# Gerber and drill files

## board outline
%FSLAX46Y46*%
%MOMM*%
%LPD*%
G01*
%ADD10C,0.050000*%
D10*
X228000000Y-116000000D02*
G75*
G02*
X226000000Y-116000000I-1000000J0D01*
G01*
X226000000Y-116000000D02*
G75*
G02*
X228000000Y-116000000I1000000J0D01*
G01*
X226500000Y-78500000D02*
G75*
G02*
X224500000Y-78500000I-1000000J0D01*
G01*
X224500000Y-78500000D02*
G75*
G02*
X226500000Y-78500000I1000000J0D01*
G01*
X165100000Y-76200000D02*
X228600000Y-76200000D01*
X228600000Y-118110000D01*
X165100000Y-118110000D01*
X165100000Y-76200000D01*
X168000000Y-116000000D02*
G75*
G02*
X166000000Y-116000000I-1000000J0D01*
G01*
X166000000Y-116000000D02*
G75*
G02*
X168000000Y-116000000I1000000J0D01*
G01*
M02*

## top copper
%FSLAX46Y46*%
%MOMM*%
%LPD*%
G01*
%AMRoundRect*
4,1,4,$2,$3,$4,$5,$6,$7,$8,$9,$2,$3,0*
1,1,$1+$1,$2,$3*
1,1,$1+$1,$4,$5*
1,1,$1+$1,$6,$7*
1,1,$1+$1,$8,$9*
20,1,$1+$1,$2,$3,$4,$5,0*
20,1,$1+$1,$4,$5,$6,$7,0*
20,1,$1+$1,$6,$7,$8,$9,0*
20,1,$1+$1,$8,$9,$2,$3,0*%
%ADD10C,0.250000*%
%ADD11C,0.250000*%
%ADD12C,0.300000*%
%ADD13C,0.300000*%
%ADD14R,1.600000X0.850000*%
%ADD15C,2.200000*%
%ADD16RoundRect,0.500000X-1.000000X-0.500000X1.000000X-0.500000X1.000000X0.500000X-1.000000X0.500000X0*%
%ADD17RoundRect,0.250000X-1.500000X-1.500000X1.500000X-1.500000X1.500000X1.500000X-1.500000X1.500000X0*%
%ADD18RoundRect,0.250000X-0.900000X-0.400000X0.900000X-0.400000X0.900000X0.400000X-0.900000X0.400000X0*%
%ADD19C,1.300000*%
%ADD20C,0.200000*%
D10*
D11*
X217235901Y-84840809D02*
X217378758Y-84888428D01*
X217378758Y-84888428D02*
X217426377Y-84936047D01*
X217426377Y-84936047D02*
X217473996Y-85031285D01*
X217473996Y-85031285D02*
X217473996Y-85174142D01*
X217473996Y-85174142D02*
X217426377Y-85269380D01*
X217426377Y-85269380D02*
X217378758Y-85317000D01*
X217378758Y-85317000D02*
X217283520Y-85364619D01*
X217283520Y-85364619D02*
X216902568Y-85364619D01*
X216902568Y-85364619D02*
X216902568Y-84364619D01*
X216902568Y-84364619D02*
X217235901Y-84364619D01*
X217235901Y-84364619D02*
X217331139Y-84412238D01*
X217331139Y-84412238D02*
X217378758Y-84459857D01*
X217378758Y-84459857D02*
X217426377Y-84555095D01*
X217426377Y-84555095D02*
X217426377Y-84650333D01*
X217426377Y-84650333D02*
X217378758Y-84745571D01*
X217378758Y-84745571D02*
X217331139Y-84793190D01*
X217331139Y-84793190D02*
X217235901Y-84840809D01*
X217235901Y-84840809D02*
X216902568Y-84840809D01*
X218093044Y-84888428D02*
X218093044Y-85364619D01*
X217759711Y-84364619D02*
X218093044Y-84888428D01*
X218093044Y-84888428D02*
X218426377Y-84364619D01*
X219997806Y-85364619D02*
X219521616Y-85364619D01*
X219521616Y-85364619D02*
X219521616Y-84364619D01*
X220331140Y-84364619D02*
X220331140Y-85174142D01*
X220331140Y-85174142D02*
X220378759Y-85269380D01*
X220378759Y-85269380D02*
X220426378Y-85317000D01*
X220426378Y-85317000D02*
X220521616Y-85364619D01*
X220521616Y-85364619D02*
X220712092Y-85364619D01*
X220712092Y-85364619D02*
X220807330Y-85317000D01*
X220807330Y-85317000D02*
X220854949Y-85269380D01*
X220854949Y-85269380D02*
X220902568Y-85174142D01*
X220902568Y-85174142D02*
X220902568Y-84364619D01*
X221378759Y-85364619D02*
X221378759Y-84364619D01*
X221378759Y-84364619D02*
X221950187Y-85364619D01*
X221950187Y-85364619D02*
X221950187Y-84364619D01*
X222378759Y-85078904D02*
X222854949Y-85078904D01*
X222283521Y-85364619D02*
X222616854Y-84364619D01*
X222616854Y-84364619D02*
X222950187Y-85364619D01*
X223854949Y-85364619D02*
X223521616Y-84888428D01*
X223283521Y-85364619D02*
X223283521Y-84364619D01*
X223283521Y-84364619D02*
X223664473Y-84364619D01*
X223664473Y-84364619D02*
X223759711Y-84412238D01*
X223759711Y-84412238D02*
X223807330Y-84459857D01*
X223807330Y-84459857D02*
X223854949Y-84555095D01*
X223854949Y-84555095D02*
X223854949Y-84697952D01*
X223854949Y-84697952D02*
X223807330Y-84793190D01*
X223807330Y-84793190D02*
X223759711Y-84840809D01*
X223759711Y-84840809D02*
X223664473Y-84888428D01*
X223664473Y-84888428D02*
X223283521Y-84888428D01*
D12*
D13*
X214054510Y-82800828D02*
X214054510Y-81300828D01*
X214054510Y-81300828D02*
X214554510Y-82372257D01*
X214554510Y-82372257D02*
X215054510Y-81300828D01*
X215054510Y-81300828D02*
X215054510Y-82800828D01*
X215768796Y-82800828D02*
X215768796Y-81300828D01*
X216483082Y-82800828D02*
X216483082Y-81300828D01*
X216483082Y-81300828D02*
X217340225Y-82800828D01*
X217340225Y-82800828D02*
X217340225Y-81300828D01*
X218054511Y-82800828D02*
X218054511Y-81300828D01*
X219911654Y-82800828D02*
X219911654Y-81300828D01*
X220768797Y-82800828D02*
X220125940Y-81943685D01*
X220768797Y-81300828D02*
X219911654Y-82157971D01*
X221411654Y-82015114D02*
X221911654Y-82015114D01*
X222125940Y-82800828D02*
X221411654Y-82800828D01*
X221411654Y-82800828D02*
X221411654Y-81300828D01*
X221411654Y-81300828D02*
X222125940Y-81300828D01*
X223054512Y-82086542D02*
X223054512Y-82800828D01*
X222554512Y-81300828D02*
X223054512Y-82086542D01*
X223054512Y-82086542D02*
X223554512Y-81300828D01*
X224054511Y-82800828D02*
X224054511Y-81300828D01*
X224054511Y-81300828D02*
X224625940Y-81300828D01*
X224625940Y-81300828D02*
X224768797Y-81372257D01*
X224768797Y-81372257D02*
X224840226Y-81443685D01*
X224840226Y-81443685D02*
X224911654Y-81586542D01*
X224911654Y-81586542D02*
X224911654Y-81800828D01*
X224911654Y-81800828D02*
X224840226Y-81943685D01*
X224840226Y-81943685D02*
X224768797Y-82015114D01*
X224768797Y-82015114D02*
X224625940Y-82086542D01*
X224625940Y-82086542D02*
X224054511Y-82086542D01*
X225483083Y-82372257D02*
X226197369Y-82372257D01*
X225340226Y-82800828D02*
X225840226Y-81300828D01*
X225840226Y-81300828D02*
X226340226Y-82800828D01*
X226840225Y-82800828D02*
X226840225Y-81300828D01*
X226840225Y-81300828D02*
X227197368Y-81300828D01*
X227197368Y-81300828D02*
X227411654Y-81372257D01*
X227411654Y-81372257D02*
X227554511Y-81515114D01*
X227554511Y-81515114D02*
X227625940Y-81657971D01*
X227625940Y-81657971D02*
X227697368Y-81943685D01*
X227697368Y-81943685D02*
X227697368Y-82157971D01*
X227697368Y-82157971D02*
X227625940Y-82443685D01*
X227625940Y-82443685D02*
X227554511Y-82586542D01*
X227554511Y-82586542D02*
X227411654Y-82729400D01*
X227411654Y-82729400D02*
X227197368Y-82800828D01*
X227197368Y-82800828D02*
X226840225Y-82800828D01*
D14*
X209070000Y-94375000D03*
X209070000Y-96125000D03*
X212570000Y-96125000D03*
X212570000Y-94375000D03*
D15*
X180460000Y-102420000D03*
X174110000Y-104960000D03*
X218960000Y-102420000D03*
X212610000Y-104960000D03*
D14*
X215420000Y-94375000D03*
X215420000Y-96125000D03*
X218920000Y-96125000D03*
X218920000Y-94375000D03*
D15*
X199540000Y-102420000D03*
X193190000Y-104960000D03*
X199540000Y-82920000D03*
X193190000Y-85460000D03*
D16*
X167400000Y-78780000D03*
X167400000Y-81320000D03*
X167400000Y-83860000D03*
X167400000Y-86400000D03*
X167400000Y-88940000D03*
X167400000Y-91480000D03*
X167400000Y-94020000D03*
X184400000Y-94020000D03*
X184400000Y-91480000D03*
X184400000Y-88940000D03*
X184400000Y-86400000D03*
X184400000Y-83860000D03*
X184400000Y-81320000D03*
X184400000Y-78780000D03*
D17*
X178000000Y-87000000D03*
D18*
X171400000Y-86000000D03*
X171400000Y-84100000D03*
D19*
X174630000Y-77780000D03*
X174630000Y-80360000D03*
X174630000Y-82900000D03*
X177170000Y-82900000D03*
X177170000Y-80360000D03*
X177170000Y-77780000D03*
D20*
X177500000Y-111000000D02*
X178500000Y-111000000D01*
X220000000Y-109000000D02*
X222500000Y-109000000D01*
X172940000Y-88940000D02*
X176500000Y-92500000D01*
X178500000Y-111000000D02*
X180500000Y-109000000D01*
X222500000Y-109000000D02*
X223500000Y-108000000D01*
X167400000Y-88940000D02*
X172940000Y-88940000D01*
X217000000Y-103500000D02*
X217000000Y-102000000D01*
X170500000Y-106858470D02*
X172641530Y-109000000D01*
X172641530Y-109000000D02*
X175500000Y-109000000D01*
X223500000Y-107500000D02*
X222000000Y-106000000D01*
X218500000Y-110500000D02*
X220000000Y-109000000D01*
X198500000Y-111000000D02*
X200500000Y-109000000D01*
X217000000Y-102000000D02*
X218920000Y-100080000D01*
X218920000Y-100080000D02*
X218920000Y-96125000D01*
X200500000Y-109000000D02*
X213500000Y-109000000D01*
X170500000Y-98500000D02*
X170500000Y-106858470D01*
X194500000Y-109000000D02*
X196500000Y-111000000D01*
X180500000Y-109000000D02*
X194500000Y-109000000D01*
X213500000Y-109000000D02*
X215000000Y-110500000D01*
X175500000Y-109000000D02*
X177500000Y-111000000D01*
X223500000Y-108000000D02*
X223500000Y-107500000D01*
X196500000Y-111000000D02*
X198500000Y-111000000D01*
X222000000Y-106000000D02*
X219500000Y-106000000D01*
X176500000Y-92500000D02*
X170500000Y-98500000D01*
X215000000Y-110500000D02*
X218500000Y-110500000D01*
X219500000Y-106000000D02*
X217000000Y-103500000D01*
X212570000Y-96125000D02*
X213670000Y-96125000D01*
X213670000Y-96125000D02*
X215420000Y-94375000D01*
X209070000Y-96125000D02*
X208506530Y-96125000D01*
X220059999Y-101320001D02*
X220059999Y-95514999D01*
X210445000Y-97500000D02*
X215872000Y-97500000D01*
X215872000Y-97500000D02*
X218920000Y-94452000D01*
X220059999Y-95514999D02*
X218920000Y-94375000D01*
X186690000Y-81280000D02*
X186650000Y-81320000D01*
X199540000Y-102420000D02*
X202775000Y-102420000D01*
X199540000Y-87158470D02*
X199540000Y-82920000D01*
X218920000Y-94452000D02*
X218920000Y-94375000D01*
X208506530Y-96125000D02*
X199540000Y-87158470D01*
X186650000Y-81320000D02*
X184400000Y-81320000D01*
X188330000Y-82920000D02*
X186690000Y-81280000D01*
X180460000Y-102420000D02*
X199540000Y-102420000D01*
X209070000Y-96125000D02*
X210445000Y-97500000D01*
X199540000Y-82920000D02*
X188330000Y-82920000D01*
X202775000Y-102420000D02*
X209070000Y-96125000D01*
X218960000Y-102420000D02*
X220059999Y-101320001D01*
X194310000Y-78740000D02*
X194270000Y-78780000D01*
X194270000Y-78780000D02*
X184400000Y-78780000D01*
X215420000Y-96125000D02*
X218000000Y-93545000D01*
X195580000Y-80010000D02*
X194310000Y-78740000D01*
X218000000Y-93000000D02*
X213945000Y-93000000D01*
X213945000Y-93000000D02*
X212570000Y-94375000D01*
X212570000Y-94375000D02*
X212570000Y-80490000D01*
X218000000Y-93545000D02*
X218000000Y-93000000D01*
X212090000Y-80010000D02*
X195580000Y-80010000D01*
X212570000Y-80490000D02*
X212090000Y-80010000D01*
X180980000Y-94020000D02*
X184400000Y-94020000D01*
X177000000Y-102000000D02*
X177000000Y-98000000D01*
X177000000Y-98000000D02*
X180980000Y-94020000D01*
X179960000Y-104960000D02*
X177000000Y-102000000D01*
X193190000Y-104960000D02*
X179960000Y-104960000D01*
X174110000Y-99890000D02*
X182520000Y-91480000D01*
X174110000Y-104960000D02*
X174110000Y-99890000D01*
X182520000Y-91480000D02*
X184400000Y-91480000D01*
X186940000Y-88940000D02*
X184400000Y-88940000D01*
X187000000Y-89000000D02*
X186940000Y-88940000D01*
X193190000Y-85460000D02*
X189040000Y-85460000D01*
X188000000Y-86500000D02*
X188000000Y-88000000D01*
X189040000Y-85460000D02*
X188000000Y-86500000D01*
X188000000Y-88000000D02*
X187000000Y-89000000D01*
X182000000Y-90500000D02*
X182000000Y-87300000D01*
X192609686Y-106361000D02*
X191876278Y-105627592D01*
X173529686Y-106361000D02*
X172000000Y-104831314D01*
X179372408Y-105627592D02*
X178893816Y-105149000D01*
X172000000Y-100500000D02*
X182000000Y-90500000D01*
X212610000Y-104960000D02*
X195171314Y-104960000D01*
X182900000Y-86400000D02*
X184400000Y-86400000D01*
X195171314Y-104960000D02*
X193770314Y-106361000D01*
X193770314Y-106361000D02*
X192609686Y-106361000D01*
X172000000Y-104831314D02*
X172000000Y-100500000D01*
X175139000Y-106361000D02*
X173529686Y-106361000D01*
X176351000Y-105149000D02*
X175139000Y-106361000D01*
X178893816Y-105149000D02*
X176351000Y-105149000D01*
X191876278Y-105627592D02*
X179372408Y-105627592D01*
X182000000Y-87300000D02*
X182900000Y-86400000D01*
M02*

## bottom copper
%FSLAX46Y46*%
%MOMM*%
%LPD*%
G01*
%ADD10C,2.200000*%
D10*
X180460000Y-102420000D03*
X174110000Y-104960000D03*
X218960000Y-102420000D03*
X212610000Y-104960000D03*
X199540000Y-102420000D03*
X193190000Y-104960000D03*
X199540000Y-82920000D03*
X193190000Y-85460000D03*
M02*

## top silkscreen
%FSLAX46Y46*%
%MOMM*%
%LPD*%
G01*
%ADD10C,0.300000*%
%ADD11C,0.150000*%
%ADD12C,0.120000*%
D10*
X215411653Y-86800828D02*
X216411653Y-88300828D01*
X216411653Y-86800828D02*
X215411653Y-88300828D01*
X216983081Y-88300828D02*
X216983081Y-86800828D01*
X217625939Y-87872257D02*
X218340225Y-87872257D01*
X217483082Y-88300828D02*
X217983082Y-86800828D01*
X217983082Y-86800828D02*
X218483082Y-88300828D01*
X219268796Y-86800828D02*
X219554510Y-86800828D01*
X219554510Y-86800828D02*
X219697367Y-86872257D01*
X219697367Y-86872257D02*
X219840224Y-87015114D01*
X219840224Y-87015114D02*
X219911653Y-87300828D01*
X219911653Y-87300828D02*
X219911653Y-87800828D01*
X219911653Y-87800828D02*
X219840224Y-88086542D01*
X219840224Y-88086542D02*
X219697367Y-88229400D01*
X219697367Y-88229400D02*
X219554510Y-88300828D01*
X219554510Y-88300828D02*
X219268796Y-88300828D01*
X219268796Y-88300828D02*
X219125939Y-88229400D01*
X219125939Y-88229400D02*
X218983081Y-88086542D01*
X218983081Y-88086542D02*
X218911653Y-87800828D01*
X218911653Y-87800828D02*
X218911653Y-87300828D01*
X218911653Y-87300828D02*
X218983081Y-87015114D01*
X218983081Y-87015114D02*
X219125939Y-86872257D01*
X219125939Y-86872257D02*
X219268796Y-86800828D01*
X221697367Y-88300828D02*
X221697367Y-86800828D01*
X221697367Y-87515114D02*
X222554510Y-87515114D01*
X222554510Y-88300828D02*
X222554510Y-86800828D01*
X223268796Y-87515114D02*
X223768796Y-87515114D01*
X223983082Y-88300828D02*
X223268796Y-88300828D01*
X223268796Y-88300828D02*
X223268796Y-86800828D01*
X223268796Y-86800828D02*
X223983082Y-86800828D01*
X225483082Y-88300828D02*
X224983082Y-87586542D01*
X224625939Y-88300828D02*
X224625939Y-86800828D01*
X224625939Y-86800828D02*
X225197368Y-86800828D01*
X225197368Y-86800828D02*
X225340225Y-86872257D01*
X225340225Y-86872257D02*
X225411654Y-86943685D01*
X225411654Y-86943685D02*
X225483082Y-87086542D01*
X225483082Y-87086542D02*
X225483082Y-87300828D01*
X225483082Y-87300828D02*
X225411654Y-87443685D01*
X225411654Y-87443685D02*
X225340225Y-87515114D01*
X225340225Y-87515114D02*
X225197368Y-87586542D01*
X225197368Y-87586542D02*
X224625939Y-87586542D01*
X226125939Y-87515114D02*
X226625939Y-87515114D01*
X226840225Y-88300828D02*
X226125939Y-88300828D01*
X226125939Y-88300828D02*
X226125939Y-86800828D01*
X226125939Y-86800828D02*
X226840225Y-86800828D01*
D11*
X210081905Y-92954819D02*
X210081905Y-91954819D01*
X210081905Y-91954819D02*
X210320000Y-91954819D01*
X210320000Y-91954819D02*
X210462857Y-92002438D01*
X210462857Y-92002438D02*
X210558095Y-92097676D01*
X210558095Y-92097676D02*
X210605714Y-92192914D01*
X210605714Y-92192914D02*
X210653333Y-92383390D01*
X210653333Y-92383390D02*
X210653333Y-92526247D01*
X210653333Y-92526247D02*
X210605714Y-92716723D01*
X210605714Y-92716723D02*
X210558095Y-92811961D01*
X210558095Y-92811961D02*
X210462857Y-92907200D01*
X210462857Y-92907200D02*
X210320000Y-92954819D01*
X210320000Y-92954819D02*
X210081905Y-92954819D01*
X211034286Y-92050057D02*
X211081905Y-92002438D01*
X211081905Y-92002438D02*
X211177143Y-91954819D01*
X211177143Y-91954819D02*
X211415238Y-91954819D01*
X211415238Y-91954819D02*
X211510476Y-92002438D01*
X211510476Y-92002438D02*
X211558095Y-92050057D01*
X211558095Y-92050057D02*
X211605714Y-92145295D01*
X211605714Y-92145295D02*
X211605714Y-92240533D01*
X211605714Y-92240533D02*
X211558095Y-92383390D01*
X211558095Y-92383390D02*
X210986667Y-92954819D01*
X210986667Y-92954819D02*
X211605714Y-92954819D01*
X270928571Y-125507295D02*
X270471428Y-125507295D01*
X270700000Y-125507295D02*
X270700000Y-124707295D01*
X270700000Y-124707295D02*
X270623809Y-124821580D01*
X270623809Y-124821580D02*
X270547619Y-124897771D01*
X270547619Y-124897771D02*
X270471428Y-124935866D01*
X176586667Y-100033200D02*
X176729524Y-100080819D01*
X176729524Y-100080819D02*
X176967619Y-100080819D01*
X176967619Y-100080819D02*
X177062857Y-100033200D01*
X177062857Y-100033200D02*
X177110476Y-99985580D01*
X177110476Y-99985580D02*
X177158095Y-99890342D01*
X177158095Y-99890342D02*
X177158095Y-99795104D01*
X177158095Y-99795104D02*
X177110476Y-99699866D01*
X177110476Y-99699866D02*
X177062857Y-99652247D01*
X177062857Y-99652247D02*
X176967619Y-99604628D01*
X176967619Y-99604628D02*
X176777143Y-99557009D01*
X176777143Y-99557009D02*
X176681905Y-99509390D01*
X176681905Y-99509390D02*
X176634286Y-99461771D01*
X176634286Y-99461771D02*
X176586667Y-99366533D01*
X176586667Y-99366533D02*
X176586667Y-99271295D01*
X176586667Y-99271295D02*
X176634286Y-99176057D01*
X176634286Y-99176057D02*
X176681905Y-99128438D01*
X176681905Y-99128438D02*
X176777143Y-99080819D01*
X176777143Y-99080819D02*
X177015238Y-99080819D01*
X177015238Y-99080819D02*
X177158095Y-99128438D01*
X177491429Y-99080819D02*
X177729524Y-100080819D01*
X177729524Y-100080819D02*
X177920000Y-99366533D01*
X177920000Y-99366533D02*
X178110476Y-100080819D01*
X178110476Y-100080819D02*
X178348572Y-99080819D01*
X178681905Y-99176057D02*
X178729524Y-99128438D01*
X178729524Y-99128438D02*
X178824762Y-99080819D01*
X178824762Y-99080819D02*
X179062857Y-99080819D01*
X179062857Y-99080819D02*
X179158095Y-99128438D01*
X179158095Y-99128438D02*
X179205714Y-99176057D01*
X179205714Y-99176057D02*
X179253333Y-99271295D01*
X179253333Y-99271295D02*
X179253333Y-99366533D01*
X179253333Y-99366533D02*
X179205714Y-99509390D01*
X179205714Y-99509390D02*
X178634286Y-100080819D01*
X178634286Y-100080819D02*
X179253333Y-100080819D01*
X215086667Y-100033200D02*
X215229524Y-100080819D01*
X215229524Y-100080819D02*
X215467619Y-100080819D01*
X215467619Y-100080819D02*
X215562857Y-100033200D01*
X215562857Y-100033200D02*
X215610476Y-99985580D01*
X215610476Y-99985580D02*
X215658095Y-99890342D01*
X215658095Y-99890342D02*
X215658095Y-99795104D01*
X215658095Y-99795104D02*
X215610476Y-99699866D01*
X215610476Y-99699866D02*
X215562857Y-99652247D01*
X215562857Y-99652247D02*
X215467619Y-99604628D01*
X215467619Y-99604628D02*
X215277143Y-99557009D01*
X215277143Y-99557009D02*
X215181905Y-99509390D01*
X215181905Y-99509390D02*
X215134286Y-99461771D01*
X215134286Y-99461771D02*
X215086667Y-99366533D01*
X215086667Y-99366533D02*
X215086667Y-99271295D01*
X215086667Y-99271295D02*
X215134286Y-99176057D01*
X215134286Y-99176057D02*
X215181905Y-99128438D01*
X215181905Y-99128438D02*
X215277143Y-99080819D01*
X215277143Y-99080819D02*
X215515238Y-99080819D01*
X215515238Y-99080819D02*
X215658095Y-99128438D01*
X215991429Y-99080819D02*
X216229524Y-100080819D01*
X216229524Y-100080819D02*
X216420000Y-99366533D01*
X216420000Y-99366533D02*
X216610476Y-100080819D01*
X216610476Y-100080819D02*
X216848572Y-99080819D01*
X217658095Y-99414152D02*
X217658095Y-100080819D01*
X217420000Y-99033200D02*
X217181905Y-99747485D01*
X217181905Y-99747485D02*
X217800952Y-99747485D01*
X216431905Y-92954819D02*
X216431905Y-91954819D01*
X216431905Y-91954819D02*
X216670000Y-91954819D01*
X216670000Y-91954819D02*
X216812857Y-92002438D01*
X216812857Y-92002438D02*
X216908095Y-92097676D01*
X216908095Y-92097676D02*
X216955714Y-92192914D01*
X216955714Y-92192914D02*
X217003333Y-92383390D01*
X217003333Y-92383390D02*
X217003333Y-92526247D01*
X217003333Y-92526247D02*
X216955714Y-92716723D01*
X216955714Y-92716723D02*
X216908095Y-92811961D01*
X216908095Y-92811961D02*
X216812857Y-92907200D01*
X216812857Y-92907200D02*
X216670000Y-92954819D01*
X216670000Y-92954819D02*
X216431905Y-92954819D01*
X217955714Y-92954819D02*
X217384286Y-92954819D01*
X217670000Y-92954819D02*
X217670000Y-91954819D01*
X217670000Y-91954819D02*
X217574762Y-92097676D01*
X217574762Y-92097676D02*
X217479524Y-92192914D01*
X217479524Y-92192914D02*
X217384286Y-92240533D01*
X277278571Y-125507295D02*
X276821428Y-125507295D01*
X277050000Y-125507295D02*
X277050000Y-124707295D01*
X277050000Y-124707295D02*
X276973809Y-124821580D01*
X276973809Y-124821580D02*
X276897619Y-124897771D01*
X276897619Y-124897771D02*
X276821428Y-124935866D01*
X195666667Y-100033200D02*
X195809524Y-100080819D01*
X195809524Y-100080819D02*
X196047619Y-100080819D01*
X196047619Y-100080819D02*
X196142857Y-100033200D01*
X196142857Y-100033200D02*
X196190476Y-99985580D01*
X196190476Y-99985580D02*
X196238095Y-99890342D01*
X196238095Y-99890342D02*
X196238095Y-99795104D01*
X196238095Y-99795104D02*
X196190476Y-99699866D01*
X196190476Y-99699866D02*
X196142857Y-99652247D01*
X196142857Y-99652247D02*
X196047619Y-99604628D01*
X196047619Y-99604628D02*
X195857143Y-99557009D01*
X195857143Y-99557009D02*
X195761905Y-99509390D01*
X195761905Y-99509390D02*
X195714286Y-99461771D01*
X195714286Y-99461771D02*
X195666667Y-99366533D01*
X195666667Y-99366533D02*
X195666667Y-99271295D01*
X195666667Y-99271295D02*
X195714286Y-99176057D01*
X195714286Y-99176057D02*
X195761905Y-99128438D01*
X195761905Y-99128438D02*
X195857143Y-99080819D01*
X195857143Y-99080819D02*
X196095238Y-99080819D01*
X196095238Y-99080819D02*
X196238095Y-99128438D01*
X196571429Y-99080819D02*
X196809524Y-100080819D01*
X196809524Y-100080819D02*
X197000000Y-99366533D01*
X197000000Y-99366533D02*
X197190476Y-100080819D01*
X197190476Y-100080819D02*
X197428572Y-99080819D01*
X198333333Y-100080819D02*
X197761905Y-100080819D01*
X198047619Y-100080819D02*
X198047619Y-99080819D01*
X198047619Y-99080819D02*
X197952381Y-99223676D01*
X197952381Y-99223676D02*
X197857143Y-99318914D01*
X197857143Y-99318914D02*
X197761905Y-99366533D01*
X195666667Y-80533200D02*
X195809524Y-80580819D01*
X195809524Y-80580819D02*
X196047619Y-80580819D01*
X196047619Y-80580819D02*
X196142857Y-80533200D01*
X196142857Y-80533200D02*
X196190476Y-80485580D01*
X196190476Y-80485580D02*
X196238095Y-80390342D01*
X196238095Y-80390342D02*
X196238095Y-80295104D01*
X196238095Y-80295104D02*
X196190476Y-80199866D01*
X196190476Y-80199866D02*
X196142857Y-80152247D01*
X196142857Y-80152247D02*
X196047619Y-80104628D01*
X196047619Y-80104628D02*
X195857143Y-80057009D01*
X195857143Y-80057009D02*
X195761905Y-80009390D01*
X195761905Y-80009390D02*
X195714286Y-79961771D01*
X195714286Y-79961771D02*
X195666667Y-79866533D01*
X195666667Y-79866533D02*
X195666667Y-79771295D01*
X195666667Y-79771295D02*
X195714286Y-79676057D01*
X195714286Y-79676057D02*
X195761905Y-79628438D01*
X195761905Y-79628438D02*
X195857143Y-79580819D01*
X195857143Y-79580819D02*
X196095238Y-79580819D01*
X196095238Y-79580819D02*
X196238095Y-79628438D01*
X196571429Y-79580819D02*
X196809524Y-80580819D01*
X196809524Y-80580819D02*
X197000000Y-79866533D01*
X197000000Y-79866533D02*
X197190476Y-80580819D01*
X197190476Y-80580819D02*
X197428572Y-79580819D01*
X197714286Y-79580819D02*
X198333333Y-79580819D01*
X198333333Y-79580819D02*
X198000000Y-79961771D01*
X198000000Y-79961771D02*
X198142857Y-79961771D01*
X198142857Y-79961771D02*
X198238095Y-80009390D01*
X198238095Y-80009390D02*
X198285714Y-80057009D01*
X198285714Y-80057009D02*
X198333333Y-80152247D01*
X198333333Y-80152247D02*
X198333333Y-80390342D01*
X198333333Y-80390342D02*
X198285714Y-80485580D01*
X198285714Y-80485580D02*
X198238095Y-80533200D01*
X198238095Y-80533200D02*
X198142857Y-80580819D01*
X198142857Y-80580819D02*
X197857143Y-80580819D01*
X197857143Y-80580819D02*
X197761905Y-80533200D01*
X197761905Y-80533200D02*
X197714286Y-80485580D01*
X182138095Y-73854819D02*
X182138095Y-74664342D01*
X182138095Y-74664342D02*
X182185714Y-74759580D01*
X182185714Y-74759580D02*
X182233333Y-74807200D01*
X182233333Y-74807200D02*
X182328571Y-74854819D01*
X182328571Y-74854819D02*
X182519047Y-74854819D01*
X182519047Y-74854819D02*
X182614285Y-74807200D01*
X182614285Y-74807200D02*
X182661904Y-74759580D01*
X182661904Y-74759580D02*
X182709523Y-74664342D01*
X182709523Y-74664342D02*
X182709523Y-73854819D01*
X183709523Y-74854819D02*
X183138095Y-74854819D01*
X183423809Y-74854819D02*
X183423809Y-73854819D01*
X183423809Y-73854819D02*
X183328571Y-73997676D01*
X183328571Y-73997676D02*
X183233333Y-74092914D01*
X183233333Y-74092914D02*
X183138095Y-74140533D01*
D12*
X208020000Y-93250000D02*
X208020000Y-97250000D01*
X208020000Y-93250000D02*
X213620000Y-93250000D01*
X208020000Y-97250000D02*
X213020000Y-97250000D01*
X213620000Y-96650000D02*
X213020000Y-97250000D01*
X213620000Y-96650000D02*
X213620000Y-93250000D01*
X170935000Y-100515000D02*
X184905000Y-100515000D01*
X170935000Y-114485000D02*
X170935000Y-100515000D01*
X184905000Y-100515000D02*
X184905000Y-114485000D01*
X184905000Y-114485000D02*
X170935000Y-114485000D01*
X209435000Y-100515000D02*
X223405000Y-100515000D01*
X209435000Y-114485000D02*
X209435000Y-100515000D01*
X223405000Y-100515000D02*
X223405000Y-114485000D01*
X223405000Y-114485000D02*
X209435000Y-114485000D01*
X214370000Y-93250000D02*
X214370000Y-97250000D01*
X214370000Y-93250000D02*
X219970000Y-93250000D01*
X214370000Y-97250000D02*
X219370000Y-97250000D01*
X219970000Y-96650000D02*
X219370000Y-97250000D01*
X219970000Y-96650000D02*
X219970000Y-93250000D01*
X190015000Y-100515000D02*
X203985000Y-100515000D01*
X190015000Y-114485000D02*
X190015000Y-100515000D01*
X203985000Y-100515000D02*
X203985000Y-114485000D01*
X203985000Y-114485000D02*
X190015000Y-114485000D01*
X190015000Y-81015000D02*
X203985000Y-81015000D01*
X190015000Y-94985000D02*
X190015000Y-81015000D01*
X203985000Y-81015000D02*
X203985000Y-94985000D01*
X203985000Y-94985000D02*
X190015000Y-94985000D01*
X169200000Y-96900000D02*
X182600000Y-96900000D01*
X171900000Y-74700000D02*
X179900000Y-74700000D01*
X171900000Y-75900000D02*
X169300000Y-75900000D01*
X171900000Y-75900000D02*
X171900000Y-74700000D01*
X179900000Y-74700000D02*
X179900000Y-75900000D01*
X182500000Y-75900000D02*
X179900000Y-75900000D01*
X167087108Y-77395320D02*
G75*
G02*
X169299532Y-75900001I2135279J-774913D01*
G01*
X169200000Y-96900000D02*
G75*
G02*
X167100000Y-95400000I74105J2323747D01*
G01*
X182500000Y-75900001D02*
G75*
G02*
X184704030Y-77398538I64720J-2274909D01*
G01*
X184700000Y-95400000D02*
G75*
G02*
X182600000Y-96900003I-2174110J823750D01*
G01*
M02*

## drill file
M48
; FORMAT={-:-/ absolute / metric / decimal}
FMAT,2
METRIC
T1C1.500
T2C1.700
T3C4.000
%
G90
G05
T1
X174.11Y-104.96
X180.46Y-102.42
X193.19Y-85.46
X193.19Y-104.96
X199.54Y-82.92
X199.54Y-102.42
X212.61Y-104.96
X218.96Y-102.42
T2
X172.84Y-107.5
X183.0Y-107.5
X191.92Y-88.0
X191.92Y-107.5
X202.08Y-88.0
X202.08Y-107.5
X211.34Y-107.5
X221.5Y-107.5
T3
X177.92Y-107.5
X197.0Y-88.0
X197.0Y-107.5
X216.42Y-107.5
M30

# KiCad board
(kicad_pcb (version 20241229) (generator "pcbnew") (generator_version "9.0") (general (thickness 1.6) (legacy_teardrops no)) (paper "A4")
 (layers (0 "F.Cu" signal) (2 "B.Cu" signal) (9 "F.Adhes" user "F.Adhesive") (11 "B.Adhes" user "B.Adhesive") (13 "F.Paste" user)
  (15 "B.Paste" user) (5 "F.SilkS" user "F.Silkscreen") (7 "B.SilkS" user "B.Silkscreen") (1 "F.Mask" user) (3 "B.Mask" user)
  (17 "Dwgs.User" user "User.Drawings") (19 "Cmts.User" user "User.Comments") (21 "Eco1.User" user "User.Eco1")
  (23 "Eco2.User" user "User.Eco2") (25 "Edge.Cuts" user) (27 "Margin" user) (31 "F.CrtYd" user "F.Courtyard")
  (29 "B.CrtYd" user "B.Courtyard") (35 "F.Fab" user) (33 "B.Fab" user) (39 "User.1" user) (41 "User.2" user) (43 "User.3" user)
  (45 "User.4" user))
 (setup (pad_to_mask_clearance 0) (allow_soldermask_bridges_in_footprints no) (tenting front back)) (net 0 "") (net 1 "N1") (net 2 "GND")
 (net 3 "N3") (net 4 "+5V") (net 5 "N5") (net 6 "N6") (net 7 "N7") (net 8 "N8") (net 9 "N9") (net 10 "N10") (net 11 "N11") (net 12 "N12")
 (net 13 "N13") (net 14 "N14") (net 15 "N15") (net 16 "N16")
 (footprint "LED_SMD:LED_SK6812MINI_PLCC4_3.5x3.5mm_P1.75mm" (layer "F.Cu") (at 210.82 95.25)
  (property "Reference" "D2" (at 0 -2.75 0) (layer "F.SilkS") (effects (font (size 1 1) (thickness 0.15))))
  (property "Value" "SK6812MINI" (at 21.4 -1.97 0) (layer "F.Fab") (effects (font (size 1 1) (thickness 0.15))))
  (fp_line (start -2.8 -2) (end -2.8 2) (stroke (width 0.12) (type default)) (layer "F.SilkS"))
  (fp_line (start -2.8 -2) (end 2.8 -2) (stroke (width 0.12) (type solid)) (layer "F.SilkS"))
  (fp_line (start -2.8 2) (end 2.2 2) (stroke (width 0.12) (type solid)) (layer "F.SilkS"))
  (fp_line (start 2.8 1.4) (end 2.2 2) (stroke (width 0.12) (type default)) (layer "F.SilkS"))
  (fp_line (start 2.8 1.4) (end 2.8 -2) (stroke (width 0.12) (type solid)) (layer "F.SilkS"))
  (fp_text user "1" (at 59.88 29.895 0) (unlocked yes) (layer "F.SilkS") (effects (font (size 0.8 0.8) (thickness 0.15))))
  (pad "1" smd rect (at -1.75 -0.875) (size 1.6 0.85) (layers "F.Cu" "F.Mask" "F.Paste") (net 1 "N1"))
  (pad "2" smd rect (at -1.75 0.875) (size 1.6 0.85) (layers "F.Cu" "F.Mask" "F.Paste") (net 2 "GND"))
  (pad "3" smd rect (at 1.75 0.875) (size 1.6 0.85) (layers "F.Cu" "F.Mask" "F.Paste") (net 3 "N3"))
  (pad "4" smd rect (at 1.75 -0.875) (size 1.6 0.85) (layers "F.Cu" "F.Mask" "F.Paste") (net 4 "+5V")))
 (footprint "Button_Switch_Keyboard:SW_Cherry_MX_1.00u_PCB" (layer "F.Cu") (at 180.46 102.42)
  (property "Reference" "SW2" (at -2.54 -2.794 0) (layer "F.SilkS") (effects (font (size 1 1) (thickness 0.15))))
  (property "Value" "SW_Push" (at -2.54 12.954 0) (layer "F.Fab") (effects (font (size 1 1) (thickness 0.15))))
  (fp_line (start -9.525 -1.905) (end 4.445 -1.905) (stroke (width 0.12) (type solid)) (layer "F.SilkS"))
  (fp_line (start -9.525 12.065) (end -9.525 -1.905) (stroke (width 0.12) (type solid)) (layer "F.SilkS"))
  (fp_line (start 4.445 -1.905) (end 4.445 12.065) (stroke (width 0.12) (type solid)) (layer "F.SilkS"))
  (fp_line (start 4.445 12.065) (end -9.525 12.065) (stroke (width 0.12) (type solid)) (layer "F.SilkS"))
  (pad "" np_thru_hole circle (at -7.62 5.08) (size 1.7 1.7) (drill 1.7) (layers "*.Cu" "*.Mask"))
  (pad "" np_thru_hole circle (at -2.54 5.08) (size 4 4) (drill 4) (layers "*.Cu" "*.Mask"))
  (pad "" np_thru_hole circle (at 2.54 5.08) (size 1.7 1.7) (drill 1.7) (layers "*.Cu" "*.Mask"))
  (pad "1" thru_hole circle (at 0 0) (size 2.2 2.2) (drill 1.5) (layers "*.Cu" "*.Mask") (remove_unused_layers no) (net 2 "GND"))
  (pad "2" thru_hole circle (at -6.35 2.54) (size 2.2 2.2) (drill 1.5) (layers "*.Cu" "*.Mask") (remove_unused_layers no) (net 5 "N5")))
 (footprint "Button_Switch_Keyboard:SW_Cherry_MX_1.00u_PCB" (layer "F.Cu") (at 218.96 102.42)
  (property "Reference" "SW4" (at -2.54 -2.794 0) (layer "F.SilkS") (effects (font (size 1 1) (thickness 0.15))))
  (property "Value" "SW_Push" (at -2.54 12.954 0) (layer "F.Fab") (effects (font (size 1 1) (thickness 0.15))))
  (fp_line (start -9.525 -1.905) (end 4.445 -1.905) (stroke (width 0.12) (type solid)) (layer "F.SilkS"))
  (fp_line (start -9.525 12.065) (end -9.525 -1.905) (stroke (width 0.12) (type solid)) (layer "F.SilkS"))
  (fp_line (start 4.445 -1.905) (end 4.445 12.065) (stroke (width 0.12) (type solid)) (layer "F.SilkS"))
  (fp_line (start 4.445 12.065) (end -9.525 12.065) (stroke (width 0.12) (type solid)) (layer "F.SilkS"))
  (pad "" np_thru_hole circle (at -7.62 5.08) (size 1.7 1.7) (drill 1.7) (layers "*.Cu" "*.Mask"))
  (pad "" np_thru_hole circle (at -2.54 5.08) (size 4 4) (drill 4) (layers "*.Cu" "*.Mask"))
  (pad "" np_thru_hole circle (at 2.54 5.08) (size 1.7 1.7) (drill 1.7) (layers "*.Cu" "*.Mask"))
  (pad "1" thru_hole circle (at 0 0) (size 2.2 2.2) (drill 1.5) (layers "*.Cu" "*.Mask") (remove_unused_layers no) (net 2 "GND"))
  (pad "2" thru_hole circle (at -6.35 2.54) (size 2.2 2.2) (drill 1.5) (layers "*.Cu" "*.Mask") (remove_unused_layers no) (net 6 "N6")))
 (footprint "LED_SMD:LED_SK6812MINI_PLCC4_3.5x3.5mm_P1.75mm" (layer "F.Cu") (at 217.17 95.25)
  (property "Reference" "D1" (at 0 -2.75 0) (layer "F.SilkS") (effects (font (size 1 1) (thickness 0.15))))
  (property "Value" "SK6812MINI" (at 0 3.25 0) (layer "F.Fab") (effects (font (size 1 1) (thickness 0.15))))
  (fp_line (start -2.8 -2) (end -2.8 2) (stroke (width 0.12) (type default)) (layer "F.SilkS"))
  (fp_line (start -2.8 -2) (end 2.8 -2) (stroke (width 0.12) (type solid)) (layer "F.SilkS"))
  (fp_line (start -2.8 2) (end 2.2 2) (stroke (width 0.12) (type solid)) (layer "F.SilkS"))
  (fp_line (start 2.8 1.4) (end 2.2 2) (stroke (width 0.12) (type default)) (layer "F.SilkS"))
  (fp_line (start 2.8 1.4) (end 2.8 -2) (stroke (width 0.12) (type solid)) (layer "F.SilkS"))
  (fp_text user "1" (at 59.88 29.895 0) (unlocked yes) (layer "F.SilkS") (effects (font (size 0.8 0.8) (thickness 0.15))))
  (pad "1" smd rect (at -1.75 -0.875) (size 1.6 0.85) (layers "F.Cu" "F.Mask" "F.Paste") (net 3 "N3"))
  (pad "2" smd rect (at -1.75 0.875) (size 1.6 0.85) (layers "F.Cu" "F.Mask" "F.Paste") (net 4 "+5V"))
  (pad "3" smd rect (at 1.75 0.875) (size 1.6 0.85) (layers "F.Cu" "F.Mask" "F.Paste") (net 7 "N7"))
  (pad "4" smd rect (at 1.75 -0.875) (size 1.6 0.85) (layers "F.Cu" "F.Mask" "F.Paste") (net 2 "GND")))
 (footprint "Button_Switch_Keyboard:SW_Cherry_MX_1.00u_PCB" (layer "F.Cu") (at 199.54 102.42)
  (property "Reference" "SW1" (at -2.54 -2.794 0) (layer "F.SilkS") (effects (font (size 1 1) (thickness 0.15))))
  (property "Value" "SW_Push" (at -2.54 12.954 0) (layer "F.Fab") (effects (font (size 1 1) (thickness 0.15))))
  (fp_line (start -9.525 -1.905) (end 4.445 -1.905) (stroke (width 0.12) (type solid)) (layer "F.SilkS"))
  (fp_line (start -9.525 12.065) (end -9.525 -1.905) (stroke (width 0.12) (type solid)) (layer "F.SilkS"))
  (fp_line (start 4.445 -1.905) (end 4.445 12.065) (stroke (width 0.12) (type solid)) (layer "F.SilkS"))
  (fp_line (start 4.445 12.065) (end -9.525 12.065) (stroke (width 0.12) (type solid)) (layer "F.SilkS"))
  (pad "" np_thru_hole circle (at -7.62 5.08) (size 1.7 1.7) (drill 1.7) (layers "*.Cu" "*.Mask"))
  (pad "" np_thru_hole circle (at -2.54 5.08) (size 4 4) (drill 4) (layers "*.Cu" "*.Mask"))
  (pad "" np_thru_hole circle (at 2.54 5.08) (size 1.7 1.7) (drill 1.7) (layers "*.Cu" "*.Mask"))
  (pad "1" thru_hole circle (at 0 0) (size 2.2 2.2) (drill 1.5) (layers "*.Cu" "*.Mask") (remove_unused_layers no) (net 2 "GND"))
  (pad "2" thru_hole circle (at -6.35 2.54) (size 2.2 2.2) (drill 1.5) (layers "*.Cu" "*.Mask") (remove_unused_layers no) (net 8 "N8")))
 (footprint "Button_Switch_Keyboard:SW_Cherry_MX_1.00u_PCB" (layer "F.Cu") (at 199.54 82.92)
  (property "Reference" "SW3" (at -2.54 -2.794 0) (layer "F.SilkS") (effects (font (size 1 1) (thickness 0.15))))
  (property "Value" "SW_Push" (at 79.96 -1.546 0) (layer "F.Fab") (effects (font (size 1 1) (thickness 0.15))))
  (fp_line (start -9.525 -1.905) (end 4.445 -1.905) (stroke (width 0.12) (type solid)) (layer "F.SilkS"))
  (fp_line (start -9.525 12.065) (end -9.525 -1.905) (stroke (width 0.12) (type solid)) (layer "F.SilkS"))
  (fp_line (start 4.445 -1.905) (end 4.445 12.065) (stroke (width 0.12) (type solid)) (layer "F.SilkS"))
  (fp_line (start 4.445 12.065) (end -9.525 12.065) (stroke (width 0.12) (type solid)) (layer "F.SilkS"))
  (pad "" np_thru_hole circle (at -7.62 5.08) (size 1.7 1.7) (drill 1.7) (layers "*.Cu" "*.Mask"))
  (pad "" np_thru_hole circle (at -2.54 5.08) (size 4 4) (drill 4) (layers "*.Cu" "*.Mask"))
  (pad "" np_thru_hole circle (at 2.54 5.08) (size 1.7 1.7) (drill 1.7) (layers "*.Cu" "*.Mask"))
  (pad "1" thru_hole circle (at 0 0) (size 2.2 2.2) (drill 1.5) (layers "*.Cu" "*.Mask") (remove_unused_layers no) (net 2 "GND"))
  (pad "2" thru_hole circle (at -6.35 2.54) (size 2.2 2.2) (drill 1.5) (layers "*.Cu" "*.Mask") (remove_unused_layers no) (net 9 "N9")))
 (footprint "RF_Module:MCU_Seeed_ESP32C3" (layer "F.Cu") (at 175.9 86.4)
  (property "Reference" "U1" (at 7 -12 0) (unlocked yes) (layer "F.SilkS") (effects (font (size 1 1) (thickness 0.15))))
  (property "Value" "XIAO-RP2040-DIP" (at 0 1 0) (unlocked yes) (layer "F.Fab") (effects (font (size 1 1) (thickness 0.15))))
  (fp_line (start -6.7 10.5) (end 6.7 10.5) (stroke (width 0.12) (type default)) (layer "F.SilkS"))
  (fp_line (start -4 -11.7) (end 4 -11.7) (stroke (width 0.12) (type default)) (layer "F.SilkS"))
  (fp_line (start -4 -10.5) (end -6.6 -10.5) (stroke (width 0.12) (type default)) (layer "F.SilkS"))
  (fp_line (start -4 -10.5) (end -4 -11.7) (stroke (width 0.12) (type default)) (layer "F.SilkS"))
  (fp_line (start 4 -11.7) (end 4 -10.5) (stroke (width 0.12) (type default)) (layer "F.SilkS"))
  (fp_line (start 6.6 -10.5) (end 4 -10.5) (stroke (width 0.12) (type default)) (layer "F.SilkS"))
  (fp_arc (start -8.812892 -9.00468) (mid -7.949609 -10.111769) (end -6.600468 -10.499999) (stroke (width 0.12) (type default))
   (layer "F.SilkS"))
  (fp_arc (start -6.7 10.5) (mid -7.977232 10.068125) (end -8.8 9) (stroke (width 0.12) (type default)) (layer "F.SilkS"))
  (fp_arc (start 6.6 -10.499999) (mid 7.944325 -10.107116) (end 8.804034 -9.001464) (stroke (width 0.12) (type default)) (layer "F.SilkS"))
  (fp_arc (start 8.8 9) (mid 7.977232 10.068125) (end 6.7 10.5) (stroke (width 0.12) (type default)) (layer "F.SilkS"))
  (pad "" smd roundrect (at 1.1 -0.4) (size 1.5 1.5) (layers "F.Paste") (roundrect_rratio 0.1666666667))
  (pad "" smd roundrect (at 1.1 1.6) (size 1.5 1.5) (layers "F.Paste") (roundrect_rratio 0.1666666667))
  (pad "" smd roundrect (at 3.1 -0.4) (size 1.5 1.5) (layers "F.Paste") (roundrect_rratio 0.1666666667))
  (pad "" smd roundrect (at 3.1 1.6) (size 1.5 1.5) (layers "F.Paste") (roundrect_rratio 0.1666666667))
  (pad "1" smd roundrect (at -8.5 -7.62) (size 3 2) (layers "F.Cu" "F.Mask" "F.Paste") (roundrect_rratio 0.25) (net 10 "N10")
   (thermal_bridge_angle 45))
  (pad "2" smd roundrect (at -8.5 -5.08) (size 3 2) (layers "F.Cu" "F.Mask" "F.Paste") (roundrect_rratio 0.25) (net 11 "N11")
   (thermal_bridge_angle 45))
  (pad "3" smd roundrect (at -8.5 -2.54) (size 3 2) (layers "F.Cu" "F.Mask" "F.Paste") (roundrect_rratio 0.25) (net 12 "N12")
   (thermal_bridge_angle 45))
  (pad "4" smd roundrect (at -8.5 0) (size 3 2) (layers "F.Cu" "F.Mask" "F.Paste") (roundrect_rratio 0.25) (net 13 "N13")
   (thermal_bridge_angle 45))
  (pad "5" smd roundrect (at -8.5 2.54) (size 3 2) (layers "F.Cu" "F.Mask" "F.Paste") (roundrect_rratio 0.25) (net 7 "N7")
   (thermal_bridge_angle 45))
  (pad "6" smd roundrect (at -8.5 5.08) (size 3 2) (layers "F.Cu" "F.Mask" "F.Paste") (roundrect_rratio 0.25) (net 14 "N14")
   (thermal_bridge_angle 45))
  (pad "7" smd roundrect (at -8.5 7.62) (size 3 2) (layers "F.Cu" "F.Mask" "F.Paste") (roundrect_rratio 0.25) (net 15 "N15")
   (thermal_bridge_angle 45))
  (pad "8" smd roundrect (at 8.5 7.62) (size 3 2) (layers "F.Cu" "F.Mask" "F.Paste") (roundrect_rratio 0.25) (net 8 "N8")
   (thermal_bridge_angle 45))
  (pad "9" smd roundrect (at 8.5 5.08) (size 3 2) (layers "F.Cu" "F.Mask" "F.Paste") (roundrect_rratio 0.25) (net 5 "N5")
   (thermal_bridge_angle 45))
  (pad "10" smd roundrect (at 8.5 2.54) (size 3 2) (layers "F.Cu" "F.Mask" "F.Paste") (roundrect_rratio 0.25) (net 9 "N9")
   (thermal_bridge_angle 45))
  (pad "11" smd roundrect (at 8.5 0) (size 3 2) (layers "F.Cu" "F.Mask" "F.Paste") (roundrect_rratio 0.25) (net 6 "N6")
   (thermal_bridge_angle 45))
  (pad "12" smd roundrect (at 8.5 -2.54) (size 3 2) (layers "F.Cu" "F.Mask" "F.Paste") (roundrect_rratio 0.25) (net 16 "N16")
   (thermal_bridge_angle 45))
  (pad "13" smd roundrect (at 8.5 -5.08) (size 3 2) (layers "F.Cu" "F.Mask" "F.Paste") (roundrect_rratio 0.25) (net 2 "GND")
   (thermal_bridge_angle 45))
  (pad "14" smd roundrect (at 8.5 -7.62) (size 3 2) (layers "F.Cu" "F.Mask" "F.Paste") (roundrect_rratio 0.25) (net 4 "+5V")
   (thermal_bridge_angle 45))
  (pad "15" smd roundrect (at 2.1 0.6) (size 3.5 3.5) (layers "F.Cu" "F.Mask") (roundrect_rratio 0.07142857143))
  (pad "16" smd roundrect (at -4.5 -0.4) (size 2.3 1.3) (layers "F.Cu" "F.Mask" "F.Paste") (roundrect_rratio 0.1923076923))
  (pad "17" smd roundrect (at -4.5 -2.3) (size 2.3 1.3) (layers "F.Cu" "F.Mask" "F.Paste") (roundrect_rratio 0.1923076923))
  (pad "18" smd circle (at -1.27 -8.62) (size 1.3 1.3) (layers "F.Cu" "F.Mask" "F.Paste"))
  (pad "19" smd circle (at -1.27 -6.04) (size 1.3 1.3) (layers "F.Cu" "F.Mask" "F.Paste"))
  (pad "20" smd circle (at -1.27 -3.5) (size 1.3 1.3) (layers "F.Cu" "F.Mask" "F.Paste"))
  (pad "21" smd circle (at 1.27 -3.5) (size 1.3 1.3) (layers "F.Cu" "F.Mask" "F.Paste"))
  (pad "22" smd circle (at 1.27 -6.04) (size 1.3 1.3) (layers "F.Cu" "F.Mask" "F.Paste"))
  (pad "23" smd circle (at 1.27 -8.62) (size 1.3 1.3) (layers "F.Cu" "F.Mask" "F.Paste")))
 (gr_circle (center 227 116) (end 228 116) (stroke (width 0.05) (type default)) (fill no) (layer "Edge.Cuts"))
 (gr_circle (center 225.5 78.5) (end 226.5 78.5) (stroke (width 0.05) (type default)) (fill no) (layer "Edge.Cuts"))
 (gr_rect (start 165.1 76.2) (end 228.6 118.11) (stroke (width 0.05) (type default)) (fill no) (layer "Edge.Cuts"))
 (gr_circle (center 167 116) (end 168 116) (stroke (width 0.05) (type default)) (fill no) (layer "Edge.Cuts"))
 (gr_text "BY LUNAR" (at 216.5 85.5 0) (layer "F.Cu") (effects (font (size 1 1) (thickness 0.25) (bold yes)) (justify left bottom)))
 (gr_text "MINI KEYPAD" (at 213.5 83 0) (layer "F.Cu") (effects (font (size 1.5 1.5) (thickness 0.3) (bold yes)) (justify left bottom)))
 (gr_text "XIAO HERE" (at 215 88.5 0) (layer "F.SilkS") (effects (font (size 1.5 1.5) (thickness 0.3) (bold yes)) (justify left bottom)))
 (segment (start 177.5 111) (end 178.5 111) (width 0.2) (layer "F.Cu") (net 7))
 (segment (start 220 109) (end 222.5 109) (width 0.2) (layer "F.Cu") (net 7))
 (segment (start 172.94 88.94) (end 176.5 92.5) (width 0.2) (layer "F.Cu") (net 7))
 (segment (start 178.5 111) (end 180.5 109) (width 0.2) (layer "F.Cu") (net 7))
 (segment (start 222.5 109) (end 223.5 108) (width 0.2) (layer "F.Cu") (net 7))
 (segment (start 167.4 88.94) (end 172.94 88.94) (width 0.2) (layer "F.Cu") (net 7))
 (segment (start 217 103.5) (end 217 102) (width 0.2) (layer "F.Cu") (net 7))
 (segment (start 170.5 106.85847) (end 172.64153 109) (width 0.2) (layer "F.Cu") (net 7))
 (segment (start 172.64153 109) (end 175.5 109) (width 0.2) (layer "F.Cu") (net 7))
 (segment (start 223.5 107.5) (end 222 106) (width 0.2) (layer "F.Cu") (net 7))
 (segment (start 218.5 110.5) (end 220 109) (width 0.2) (layer "F.Cu") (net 7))
 (segment (start 198.5 111) (end 200.5 109) (width 0.2) (layer "F.Cu") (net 7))
 (segment (start 217 102) (end 218.92 100.08) (width 0.2) (layer "F.Cu") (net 7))
 (segment (start 218.92 100.08) (end 218.92 96.125) (width 0.2) (layer "F.Cu") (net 7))
 (segment (start 200.5 109) (end 213.5 109) (width 0.2) (layer "F.Cu") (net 7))
 (segment (start 170.5 98.5) (end 170.5 106.85847) (width 0.2) (layer "F.Cu") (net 7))
 (segment (start 194.5 109) (end 196.5 111) (width 0.2) (layer "F.Cu") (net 7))
 (segment (start 180.5 109) (end 194.5 109) (width 0.2) (layer "F.Cu") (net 7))
 (segment (start 213.5 109) (end 215 110.5) (width 0.2) (layer "F.Cu") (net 7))
 (segment (start 175.5 109) (end 177.5 111) (width 0.2) (layer "F.Cu") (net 7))
 (segment (start 223.5 108) (end 223.5 107.5) (width 0.2) (layer "F.Cu") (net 7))
 (segment (start 196.5 111) (end 198.5 111) (width 0.2) (layer "F.Cu") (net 7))
 (segment (start 222 106) (end 219.5 106) (width 0.2) (layer "F.Cu") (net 7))
 (segment (start 176.5 92.5) (end 170.5 98.5) (width 0.2) (layer "F.Cu") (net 7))
 (segment (start 215 110.5) (end 218.5 110.5) (width 0.2) (layer "F.Cu") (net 7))
 (segment (start 219.5 106) (end 217 103.5) (width 0.2) (layer "F.Cu") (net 7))
 (segment (start 212.57 96.125) (end 213.67 96.125) (width 0.2) (layer "F.Cu") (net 3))
 (segment (start 213.67 96.125) (end 215.42 94.375) (width 0.2) (layer "F.Cu") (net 3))
 (segment (start 209.07 96.125) (end 208.50653 96.125) (width 0.2) (layer "F.Cu") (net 2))
 (segment (start 220.059999 101.320001) (end 220.059999 95.514999) (width 0.2) (layer "F.Cu") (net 2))
 (segment (start 210.445 97.5) (end 215.872 97.5) (width 0.2) (layer "F.Cu") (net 2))
 (segment (start 215.872 97.5) (end 218.92 94.452) (width 0.2) (layer "F.Cu") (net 2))
 (segment (start 220.059999 95.514999) (end 218.92 94.375) (width 0.2) (layer "F.Cu") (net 2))
 (segment (start 186.69 81.28) (end 186.65 81.32) (width 0.2) (layer "F.Cu") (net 2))
 (segment (start 199.54 102.42) (end 202.775 102.42) (width 0.2) (layer "F.Cu") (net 2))
 (segment (start 199.54 87.15847) (end 199.54 82.92) (width 0.2) (layer "F.Cu") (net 2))
 (segment (start 218.92 94.452) (end 218.92 94.375) (width 0.2) (layer "F.Cu") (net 2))
 (segment (start 208.50653 96.125) (end 199.54 87.15847) (width 0.2) (layer "F.Cu") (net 2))
 (segment (start 186.65 81.32) (end 184.4 81.32) (width 0.2) (layer "F.Cu") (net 2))
 (segment (start 188.33 82.92) (end 186.69 81.28) (width 0.2) (layer "F.Cu") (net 2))
 (segment (start 180.46 102.42) (end 199.54 102.42) (width 0.2) (layer "F.Cu") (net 2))
 (segment (start 209.07 96.125) (end 210.445 97.5) (width 0.2) (layer "F.Cu") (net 2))
 (segment (start 199.54 82.92) (end 188.33 82.92) (width 0.2) (layer "F.Cu") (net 2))
 (segment (start 202.775 102.42) (end 209.07 96.125) (width 0.2) (layer "F.Cu") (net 2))
 (segment (start 218.96 102.42) (end 220.059999 101.320001) (width 0.2) (layer "F.Cu") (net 2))
 (segment (start 194.31 78.74) (end 194.27 78.78) (width 0.2) (layer "F.Cu") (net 4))
 (segment (start 194.27 78.78) (end 184.4 78.78) (width 0.2) (layer "F.Cu") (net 4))
 (segment (start 215.42 96.125) (end 218 93.545) (width 0.2) (layer "F.Cu") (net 4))
 (segment (start 195.58 80.01) (end 194.31 78.74) (width 0.2) (layer "F.Cu") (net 4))
 (segment (start 218 93) (end 213.945 93) (width 0.2) (layer "F.Cu") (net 4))
 (segment (start 213.945 93) (end 212.57 94.375) (width 0.2) (layer "F.Cu") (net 4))
 (segment (start 212.57 94.375) (end 212.57 80.49) (width 0.2) (layer "F.Cu") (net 4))
 (segment (start 218 93.545) (end 218 93) (width 0.2) (layer "F.Cu") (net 4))
 (segment (start 212.09 80.01) (end 195.58 80.01) (width 0.2) (layer "F.Cu") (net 4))
 (segment (start 212.57 80.49) (end 212.09 80.01) (width 0.2) (layer "F.Cu") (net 4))
 (segment (start 180.98 94.02) (end 184.4 94.02) (width 0.2) (layer "F.Cu") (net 8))
 (segment (start 177 102) (end 177 98) (width 0.2) (layer "F.Cu") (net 8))
 (segment (start 177 98) (end 180.98 94.02) (width 0.2) (layer "F.Cu") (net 8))
 (segment (start 179.96 104.96) (end 177 102) (width 0.2) (layer "F.Cu") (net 8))
 (segment (start 193.19 104.96) (end 179.96 104.96) (width 0.2) (layer "F.Cu") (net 8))
 (segment (start 174.11 99.89) (end 182.52 91.48) (width 0.2) (layer "F.Cu") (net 5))
 (segment (start 174.11 104.96) (end 174.11 99.89) (width 0.2) (layer "F.Cu") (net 5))
 (segment (start 182.52 91.48) (end 184.4 91.48) (width 0.2) (layer "F.Cu") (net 5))
 (segment (start 186.94 88.94) (end 184.4 88.94) (width 0.2) (layer "F.Cu") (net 9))
 (segment (start 187 89) (end 186.94 88.94) (width 0.2) (layer "F.Cu") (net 9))
 (segment (start 193.19 85.46) (end 189.04 85.46) (width 0.2) (layer "F.Cu") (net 9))
 (segment (start 188 86.5) (end 188 88) (width 0.2) (layer "F.Cu") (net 9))
 (segment (start 189.04 85.46) (end 188 86.5) (width 0.2) (layer "F.Cu") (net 9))
 (segment (start 188 88) (end 187 89) (width 0.2) (layer "F.Cu") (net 9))
 (segment (start 182 90.5) (end 182 87.3) (width 0.2) (layer "F.Cu") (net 6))
 (segment (start 192.609686 106.361) (end 191.876278 105.627592) (width 0.2) (layer "F.Cu") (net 6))
 (segment (start 173.529686 106.361) (end 172 104.831314) (width 0.2) (layer "F.Cu") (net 6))
 (segment (start 179.372408 105.627592) (end 178.893816 105.149) (width 0.2) (layer "F.Cu") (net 6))
 (segment (start 172 100.5) (end 182 90.5) (width 0.2) (layer "F.Cu") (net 6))
 (segment (start 212.61 104.96) (end 195.171314 104.96) (width 0.2) (layer "F.Cu") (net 6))
 (segment (start 182.9 86.4) (end 184.4 86.4) (width 0.2) (layer "F.Cu") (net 6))
 (segment (start 195.171314 104.96) (end 193.770314 106.361) (width 0.2) (layer "F.Cu") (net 6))
 (segment (start 193.770314 106.361) (end 192.609686 106.361) (width 0.2) (layer "F.Cu") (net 6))
 (segment (start 172 104.831314) (end 172 100.5) (width 0.2) (layer "F.Cu") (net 6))
 (segment (start 175.139 106.361) (end 173.529686 106.361) (width 0.2) (layer "F.Cu") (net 6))
 (segment (start 176.351 105.149) (end 175.139 106.361) (width 0.2) (layer "F.Cu") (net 6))
 (segment (start 178.893816 105.149) (end 176.351 105.149) (width 0.2) (layer "F.Cu") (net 6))
 (segment (start 191.876278 105.627592) (end 179.372408 105.627592) (width 0.2) (layer "F.Cu") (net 6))
 (segment (start 182 87.3) (end 182.9 86.4) (width 0.2) (layer "F.Cu") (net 6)))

